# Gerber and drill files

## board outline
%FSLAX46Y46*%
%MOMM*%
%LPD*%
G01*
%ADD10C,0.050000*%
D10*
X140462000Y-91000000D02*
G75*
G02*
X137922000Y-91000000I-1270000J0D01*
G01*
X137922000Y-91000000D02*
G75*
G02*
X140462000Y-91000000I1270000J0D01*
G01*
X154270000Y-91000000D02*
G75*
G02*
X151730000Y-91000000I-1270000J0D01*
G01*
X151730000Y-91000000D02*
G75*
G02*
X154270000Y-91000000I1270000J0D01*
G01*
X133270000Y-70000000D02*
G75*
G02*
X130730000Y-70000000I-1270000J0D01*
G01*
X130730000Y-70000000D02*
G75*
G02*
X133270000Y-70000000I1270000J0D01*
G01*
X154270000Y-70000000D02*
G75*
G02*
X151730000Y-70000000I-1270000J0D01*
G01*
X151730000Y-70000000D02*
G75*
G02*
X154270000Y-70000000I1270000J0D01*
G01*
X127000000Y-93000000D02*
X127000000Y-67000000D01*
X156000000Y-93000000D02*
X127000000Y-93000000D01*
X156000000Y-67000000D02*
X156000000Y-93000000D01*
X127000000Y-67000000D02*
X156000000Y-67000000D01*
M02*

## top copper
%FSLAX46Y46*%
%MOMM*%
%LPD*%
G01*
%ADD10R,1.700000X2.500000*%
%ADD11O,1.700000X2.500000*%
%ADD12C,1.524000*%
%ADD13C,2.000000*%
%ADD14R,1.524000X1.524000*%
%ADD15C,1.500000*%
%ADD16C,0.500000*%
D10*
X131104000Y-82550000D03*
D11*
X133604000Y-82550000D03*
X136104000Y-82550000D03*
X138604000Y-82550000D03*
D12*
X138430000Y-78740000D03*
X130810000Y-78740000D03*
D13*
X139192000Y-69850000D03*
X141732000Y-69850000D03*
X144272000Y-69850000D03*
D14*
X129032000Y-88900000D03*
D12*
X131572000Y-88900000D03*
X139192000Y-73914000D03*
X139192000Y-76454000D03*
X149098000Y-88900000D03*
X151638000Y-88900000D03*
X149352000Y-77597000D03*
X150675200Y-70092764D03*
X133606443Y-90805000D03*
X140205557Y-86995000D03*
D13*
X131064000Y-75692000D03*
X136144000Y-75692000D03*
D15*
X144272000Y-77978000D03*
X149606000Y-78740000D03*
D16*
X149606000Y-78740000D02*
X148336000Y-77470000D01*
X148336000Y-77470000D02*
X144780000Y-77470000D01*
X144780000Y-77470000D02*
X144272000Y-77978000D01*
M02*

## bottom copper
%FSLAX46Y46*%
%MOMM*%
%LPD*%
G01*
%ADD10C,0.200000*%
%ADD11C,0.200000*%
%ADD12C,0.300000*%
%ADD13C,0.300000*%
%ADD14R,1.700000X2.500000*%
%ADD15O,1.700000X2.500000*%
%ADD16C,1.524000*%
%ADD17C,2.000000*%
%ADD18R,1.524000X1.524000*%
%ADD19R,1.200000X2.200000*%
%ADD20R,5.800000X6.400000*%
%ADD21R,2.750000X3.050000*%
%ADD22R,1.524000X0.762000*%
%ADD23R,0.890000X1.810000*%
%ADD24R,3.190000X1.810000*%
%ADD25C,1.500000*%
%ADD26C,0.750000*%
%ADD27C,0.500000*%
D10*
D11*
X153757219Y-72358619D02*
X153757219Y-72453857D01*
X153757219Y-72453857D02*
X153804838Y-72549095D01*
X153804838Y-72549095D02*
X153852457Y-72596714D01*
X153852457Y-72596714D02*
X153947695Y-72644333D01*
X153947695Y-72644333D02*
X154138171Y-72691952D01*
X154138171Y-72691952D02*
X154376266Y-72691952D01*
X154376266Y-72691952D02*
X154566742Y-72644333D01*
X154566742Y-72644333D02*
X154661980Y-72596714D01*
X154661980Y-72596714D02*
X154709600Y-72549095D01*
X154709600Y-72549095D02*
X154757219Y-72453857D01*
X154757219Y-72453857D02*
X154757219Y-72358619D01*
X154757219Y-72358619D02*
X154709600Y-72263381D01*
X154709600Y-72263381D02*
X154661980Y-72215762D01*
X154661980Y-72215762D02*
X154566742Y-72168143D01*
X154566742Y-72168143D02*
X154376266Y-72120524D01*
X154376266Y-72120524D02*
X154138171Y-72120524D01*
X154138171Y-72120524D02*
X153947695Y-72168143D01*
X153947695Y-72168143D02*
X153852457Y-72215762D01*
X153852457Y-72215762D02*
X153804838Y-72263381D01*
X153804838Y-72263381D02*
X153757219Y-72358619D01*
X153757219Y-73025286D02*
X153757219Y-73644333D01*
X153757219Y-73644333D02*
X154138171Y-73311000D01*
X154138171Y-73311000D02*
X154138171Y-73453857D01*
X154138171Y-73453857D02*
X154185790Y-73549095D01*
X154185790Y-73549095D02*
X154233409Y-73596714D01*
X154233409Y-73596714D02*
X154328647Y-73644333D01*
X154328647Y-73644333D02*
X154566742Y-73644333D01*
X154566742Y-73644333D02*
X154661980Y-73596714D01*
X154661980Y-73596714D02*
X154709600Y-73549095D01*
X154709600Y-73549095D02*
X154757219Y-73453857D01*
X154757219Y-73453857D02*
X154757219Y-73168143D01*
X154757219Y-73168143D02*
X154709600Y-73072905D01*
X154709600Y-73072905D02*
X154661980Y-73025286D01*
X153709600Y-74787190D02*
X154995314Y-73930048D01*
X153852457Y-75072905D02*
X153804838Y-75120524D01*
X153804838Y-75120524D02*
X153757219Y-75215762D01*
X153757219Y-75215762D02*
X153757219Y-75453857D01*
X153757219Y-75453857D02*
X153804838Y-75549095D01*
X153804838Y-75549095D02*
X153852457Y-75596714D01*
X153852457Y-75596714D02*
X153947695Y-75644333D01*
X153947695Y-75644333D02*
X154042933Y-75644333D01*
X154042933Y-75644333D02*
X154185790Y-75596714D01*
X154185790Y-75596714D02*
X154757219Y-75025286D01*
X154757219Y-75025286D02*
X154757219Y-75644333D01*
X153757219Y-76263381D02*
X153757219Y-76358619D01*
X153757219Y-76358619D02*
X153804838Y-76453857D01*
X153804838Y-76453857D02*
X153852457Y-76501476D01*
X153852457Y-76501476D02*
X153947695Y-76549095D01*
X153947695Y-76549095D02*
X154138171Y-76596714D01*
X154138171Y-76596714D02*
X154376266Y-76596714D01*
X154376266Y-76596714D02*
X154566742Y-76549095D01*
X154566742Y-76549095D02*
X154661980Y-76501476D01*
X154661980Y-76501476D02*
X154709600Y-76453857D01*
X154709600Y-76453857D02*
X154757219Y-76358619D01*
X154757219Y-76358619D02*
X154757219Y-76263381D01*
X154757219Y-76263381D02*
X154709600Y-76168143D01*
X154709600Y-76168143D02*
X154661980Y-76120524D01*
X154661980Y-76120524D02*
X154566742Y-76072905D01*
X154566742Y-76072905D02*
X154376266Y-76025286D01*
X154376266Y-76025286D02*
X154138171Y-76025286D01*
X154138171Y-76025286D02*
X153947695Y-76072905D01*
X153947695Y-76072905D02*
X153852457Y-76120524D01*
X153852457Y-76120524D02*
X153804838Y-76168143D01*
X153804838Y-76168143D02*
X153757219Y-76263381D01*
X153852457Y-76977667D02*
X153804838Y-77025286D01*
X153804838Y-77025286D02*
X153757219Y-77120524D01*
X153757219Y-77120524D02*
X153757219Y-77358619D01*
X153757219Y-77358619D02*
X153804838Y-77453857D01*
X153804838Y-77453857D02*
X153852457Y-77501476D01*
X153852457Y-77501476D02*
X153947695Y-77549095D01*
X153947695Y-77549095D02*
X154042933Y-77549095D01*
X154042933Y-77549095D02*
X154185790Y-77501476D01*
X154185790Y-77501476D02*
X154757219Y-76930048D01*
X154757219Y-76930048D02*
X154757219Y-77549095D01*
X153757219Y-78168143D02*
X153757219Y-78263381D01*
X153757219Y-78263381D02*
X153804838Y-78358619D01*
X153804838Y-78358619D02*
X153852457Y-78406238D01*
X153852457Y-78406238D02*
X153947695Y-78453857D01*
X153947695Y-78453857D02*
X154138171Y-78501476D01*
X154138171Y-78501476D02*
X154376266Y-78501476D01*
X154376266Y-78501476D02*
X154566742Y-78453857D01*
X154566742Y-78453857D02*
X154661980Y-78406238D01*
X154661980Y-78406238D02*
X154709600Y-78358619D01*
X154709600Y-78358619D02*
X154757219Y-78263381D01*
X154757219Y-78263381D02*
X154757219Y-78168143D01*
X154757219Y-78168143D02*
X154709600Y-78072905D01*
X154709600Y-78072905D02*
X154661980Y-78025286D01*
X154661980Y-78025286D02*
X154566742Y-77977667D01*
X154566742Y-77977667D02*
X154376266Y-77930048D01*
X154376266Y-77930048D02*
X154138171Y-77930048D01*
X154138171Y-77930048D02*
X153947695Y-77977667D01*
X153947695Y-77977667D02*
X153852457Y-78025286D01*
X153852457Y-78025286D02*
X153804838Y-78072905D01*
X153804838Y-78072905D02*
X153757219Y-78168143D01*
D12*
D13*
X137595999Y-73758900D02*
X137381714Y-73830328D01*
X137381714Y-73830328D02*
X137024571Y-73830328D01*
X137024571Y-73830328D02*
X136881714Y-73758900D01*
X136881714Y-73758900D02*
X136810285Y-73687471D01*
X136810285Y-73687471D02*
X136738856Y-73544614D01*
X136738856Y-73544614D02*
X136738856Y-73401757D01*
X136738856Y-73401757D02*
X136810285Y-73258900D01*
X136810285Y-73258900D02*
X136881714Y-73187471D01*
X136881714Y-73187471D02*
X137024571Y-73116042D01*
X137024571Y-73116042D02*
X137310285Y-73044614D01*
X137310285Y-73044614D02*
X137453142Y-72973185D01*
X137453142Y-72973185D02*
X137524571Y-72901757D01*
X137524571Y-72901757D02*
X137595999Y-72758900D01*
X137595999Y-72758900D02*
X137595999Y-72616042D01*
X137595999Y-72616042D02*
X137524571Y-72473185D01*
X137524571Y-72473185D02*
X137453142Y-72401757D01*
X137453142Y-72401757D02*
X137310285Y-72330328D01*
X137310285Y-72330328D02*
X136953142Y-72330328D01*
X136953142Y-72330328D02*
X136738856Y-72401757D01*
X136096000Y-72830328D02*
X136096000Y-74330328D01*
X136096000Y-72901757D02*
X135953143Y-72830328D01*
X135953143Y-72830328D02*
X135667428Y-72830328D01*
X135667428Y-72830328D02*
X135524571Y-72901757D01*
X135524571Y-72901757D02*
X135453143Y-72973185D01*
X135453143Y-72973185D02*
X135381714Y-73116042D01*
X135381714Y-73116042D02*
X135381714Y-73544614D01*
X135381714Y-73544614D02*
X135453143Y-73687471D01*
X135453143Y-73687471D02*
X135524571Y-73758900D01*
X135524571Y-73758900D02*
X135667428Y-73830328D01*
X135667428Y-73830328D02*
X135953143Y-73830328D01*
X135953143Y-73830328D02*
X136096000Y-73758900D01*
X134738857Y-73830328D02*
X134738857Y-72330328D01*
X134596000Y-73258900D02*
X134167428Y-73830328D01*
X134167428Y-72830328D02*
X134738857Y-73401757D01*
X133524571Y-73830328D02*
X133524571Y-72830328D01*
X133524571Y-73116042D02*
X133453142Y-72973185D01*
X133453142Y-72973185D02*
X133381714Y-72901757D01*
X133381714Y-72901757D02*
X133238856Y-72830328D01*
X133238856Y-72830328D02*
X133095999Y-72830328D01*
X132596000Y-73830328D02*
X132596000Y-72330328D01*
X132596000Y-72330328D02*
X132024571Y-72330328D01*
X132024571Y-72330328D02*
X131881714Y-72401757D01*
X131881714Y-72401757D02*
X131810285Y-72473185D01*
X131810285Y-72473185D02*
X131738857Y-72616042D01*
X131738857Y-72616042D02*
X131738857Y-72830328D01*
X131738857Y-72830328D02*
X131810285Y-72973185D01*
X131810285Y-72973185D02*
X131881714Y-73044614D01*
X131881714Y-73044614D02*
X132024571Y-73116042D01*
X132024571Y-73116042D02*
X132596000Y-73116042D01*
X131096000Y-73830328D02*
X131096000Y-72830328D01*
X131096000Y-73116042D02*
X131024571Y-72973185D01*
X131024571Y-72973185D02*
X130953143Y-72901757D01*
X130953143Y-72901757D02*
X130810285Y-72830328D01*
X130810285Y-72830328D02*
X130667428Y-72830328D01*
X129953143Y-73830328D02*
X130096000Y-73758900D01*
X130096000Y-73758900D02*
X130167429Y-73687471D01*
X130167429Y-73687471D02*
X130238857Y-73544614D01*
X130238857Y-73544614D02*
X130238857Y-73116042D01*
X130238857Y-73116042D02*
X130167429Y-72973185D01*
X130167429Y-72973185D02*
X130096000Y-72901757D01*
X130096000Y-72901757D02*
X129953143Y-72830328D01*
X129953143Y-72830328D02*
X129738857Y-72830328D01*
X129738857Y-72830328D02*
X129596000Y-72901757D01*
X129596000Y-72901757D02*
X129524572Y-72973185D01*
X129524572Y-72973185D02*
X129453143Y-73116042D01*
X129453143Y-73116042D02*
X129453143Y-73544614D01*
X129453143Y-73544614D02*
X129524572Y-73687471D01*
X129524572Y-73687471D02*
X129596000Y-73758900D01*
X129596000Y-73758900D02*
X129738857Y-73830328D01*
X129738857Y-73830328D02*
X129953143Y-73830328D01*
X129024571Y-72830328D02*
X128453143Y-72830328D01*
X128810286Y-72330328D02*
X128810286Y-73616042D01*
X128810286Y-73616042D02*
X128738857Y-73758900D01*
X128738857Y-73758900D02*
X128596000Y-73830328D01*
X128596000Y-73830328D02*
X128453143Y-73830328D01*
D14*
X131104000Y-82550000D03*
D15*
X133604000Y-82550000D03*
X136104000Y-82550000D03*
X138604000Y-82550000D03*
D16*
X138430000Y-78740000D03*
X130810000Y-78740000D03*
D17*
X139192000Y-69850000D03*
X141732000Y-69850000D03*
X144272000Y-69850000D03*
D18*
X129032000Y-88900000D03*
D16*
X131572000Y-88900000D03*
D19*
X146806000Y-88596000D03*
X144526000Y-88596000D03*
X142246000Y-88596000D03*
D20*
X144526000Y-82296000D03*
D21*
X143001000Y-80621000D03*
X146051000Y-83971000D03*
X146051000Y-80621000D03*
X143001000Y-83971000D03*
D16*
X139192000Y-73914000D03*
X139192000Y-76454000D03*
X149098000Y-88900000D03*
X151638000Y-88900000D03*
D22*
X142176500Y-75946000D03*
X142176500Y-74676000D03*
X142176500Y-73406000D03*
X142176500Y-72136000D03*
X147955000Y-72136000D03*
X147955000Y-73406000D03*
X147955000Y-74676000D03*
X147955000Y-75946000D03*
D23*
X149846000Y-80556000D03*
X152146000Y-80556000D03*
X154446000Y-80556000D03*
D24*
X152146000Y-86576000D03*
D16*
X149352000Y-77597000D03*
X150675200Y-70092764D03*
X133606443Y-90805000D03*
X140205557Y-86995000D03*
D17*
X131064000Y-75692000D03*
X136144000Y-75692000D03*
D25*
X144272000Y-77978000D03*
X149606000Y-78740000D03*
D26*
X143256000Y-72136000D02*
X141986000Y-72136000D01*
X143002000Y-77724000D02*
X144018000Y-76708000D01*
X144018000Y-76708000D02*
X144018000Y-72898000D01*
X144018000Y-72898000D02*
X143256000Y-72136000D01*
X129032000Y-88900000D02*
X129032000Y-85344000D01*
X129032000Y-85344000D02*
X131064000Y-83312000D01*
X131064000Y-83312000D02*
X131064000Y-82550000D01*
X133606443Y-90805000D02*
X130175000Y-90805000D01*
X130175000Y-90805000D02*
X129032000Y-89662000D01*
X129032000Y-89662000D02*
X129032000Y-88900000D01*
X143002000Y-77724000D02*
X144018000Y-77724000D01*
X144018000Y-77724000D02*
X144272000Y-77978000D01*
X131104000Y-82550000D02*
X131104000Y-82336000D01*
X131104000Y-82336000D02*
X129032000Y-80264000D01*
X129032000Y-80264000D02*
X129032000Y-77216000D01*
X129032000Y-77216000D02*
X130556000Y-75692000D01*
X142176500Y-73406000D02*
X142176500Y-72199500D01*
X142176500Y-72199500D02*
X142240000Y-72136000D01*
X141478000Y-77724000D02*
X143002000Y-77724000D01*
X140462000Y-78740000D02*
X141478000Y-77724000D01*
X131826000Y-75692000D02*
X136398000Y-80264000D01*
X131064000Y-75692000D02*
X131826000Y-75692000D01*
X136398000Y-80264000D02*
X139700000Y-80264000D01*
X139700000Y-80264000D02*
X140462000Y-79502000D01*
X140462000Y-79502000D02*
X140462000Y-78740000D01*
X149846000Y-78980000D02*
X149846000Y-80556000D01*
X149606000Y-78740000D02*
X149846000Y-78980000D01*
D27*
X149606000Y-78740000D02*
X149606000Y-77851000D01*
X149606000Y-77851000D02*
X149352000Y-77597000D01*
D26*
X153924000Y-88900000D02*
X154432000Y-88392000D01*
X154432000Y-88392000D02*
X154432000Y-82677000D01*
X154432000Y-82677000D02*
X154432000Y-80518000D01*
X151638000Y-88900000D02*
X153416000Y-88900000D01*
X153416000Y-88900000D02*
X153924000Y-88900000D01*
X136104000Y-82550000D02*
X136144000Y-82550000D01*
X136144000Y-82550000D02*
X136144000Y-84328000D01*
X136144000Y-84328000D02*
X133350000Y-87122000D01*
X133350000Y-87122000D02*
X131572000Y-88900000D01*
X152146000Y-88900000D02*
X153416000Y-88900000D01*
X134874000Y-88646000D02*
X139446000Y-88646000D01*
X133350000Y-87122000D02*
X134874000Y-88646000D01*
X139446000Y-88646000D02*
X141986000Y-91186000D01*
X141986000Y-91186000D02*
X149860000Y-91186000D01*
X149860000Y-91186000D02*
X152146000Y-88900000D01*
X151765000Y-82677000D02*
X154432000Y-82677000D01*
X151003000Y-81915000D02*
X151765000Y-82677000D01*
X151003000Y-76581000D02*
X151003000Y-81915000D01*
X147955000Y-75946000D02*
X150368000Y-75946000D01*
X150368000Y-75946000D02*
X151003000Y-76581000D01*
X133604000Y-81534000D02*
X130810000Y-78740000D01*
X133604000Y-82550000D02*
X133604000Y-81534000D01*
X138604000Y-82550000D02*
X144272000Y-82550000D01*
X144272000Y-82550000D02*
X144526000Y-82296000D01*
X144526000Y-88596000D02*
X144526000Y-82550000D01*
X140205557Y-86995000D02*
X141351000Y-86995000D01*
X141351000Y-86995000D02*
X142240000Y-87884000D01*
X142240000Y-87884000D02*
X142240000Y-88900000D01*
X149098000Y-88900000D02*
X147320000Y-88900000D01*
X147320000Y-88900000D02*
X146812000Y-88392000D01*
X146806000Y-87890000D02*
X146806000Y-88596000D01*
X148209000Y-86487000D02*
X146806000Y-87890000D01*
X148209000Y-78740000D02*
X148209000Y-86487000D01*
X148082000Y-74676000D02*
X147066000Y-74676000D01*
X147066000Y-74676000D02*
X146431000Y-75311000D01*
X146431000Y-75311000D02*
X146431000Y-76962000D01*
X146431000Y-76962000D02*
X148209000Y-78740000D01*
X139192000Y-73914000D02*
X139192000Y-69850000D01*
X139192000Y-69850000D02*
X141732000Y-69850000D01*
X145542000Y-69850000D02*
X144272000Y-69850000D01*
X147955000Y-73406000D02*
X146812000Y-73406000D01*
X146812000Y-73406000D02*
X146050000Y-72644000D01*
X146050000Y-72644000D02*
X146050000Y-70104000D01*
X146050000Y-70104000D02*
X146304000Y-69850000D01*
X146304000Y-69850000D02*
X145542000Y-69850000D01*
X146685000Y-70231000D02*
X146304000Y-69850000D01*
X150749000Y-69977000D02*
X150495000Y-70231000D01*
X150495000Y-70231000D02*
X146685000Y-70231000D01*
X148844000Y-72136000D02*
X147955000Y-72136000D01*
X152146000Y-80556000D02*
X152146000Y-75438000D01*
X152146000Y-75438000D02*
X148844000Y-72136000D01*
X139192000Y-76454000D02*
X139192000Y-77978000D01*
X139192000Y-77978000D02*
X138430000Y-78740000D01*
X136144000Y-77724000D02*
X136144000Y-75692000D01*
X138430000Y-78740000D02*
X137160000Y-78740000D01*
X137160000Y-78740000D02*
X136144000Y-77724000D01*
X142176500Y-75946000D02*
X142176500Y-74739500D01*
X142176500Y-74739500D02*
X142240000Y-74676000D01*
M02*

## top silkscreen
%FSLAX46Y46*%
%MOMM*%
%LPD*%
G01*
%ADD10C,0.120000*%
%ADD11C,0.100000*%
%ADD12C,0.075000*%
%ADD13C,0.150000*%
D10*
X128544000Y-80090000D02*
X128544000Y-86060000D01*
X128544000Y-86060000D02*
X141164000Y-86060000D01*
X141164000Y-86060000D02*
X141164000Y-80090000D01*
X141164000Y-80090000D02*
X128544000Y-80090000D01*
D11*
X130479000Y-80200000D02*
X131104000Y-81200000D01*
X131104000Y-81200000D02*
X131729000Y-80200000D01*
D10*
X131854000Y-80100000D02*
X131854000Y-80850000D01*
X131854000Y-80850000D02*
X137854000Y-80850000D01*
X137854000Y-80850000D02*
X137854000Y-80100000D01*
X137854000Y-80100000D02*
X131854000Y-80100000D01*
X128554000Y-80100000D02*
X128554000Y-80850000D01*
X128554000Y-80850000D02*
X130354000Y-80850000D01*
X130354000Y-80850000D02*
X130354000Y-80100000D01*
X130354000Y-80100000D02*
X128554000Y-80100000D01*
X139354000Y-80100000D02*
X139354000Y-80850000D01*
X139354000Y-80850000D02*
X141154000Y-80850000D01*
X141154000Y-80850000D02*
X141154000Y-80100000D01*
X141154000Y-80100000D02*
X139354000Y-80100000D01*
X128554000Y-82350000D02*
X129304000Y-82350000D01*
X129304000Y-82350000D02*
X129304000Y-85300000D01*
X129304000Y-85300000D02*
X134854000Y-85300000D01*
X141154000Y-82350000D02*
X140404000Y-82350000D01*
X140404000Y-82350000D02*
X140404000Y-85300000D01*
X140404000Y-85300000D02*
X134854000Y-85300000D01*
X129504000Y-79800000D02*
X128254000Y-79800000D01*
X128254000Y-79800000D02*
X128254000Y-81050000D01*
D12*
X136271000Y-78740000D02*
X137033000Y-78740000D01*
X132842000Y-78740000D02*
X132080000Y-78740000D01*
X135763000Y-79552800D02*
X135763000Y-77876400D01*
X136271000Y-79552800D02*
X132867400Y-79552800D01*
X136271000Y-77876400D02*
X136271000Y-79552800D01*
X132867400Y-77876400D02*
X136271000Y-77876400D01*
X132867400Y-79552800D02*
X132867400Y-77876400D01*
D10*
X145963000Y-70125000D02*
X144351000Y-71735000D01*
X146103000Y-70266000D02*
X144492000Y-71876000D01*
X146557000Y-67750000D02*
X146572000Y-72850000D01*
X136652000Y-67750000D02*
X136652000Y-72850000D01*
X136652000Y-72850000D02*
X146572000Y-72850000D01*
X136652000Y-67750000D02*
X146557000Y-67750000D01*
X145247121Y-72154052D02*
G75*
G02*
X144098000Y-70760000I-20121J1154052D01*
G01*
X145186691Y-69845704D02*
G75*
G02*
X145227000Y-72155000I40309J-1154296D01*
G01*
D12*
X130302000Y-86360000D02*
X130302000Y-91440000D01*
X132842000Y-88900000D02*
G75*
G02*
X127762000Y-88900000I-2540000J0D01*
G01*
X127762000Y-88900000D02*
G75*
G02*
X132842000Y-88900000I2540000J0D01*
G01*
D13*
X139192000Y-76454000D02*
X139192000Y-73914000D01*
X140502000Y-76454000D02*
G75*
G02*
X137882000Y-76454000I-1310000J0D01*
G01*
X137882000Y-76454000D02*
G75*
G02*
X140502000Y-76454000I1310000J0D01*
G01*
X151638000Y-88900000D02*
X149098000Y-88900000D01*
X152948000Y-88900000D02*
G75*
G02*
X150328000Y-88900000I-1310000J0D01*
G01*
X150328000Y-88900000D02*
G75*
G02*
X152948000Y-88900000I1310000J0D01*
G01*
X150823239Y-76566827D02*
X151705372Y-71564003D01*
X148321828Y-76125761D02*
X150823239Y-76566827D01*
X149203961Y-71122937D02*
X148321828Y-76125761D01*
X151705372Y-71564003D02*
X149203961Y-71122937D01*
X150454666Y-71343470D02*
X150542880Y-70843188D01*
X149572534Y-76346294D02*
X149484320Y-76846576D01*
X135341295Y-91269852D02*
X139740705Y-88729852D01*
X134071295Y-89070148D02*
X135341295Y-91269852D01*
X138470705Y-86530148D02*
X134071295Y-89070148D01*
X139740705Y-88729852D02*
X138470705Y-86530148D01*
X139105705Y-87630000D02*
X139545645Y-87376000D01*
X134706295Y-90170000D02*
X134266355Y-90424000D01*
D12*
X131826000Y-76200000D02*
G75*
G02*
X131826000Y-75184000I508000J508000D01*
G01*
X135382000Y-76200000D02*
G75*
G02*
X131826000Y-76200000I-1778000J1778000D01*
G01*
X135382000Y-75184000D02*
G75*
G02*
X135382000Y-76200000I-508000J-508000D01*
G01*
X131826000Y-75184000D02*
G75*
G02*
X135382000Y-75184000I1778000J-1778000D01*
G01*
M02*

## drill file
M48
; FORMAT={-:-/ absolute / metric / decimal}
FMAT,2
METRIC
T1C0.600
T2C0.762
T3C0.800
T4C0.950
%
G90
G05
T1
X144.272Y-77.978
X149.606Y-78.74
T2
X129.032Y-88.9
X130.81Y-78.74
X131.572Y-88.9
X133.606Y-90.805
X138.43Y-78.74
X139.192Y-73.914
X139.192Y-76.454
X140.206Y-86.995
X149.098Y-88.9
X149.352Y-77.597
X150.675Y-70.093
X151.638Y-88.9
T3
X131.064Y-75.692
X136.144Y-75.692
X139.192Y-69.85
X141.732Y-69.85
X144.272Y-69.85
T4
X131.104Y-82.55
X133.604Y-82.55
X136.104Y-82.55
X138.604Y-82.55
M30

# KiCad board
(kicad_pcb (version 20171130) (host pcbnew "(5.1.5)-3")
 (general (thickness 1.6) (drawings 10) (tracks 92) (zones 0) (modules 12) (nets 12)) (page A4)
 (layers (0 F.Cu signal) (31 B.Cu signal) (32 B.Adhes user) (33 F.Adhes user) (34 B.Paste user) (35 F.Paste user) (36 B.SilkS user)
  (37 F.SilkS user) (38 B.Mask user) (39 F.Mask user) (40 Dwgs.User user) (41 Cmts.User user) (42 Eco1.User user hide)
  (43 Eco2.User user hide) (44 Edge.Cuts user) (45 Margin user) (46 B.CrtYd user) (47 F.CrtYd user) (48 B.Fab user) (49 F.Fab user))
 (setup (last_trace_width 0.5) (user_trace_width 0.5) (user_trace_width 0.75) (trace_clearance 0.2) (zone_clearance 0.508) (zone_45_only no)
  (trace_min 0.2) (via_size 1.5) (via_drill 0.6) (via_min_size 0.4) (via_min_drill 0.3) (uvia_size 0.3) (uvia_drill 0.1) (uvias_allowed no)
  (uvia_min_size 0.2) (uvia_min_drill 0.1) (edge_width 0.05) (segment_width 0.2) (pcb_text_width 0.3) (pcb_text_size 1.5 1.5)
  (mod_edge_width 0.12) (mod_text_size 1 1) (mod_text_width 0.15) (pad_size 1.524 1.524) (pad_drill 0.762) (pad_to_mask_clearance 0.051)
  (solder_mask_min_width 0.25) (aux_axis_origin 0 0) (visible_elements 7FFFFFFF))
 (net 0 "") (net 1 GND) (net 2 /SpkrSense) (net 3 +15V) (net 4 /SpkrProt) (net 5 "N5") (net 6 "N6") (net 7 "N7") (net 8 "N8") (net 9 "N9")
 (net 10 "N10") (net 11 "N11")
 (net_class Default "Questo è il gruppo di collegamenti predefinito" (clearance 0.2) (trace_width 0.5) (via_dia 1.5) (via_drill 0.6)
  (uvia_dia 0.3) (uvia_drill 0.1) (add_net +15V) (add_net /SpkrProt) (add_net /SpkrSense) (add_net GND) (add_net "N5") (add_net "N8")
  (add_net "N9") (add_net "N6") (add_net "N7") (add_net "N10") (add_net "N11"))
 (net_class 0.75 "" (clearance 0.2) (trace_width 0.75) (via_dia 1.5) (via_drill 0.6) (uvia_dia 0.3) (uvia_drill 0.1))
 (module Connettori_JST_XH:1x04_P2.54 (layer F.Cu) (at 131.104 82.55)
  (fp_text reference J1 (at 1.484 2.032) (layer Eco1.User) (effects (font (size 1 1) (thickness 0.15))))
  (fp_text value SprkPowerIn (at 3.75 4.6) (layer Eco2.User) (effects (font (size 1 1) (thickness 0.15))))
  (fp_line (start -2.56 -2.46) (end -2.56 3.51) (layer F.SilkS) (width 0.12))
  (fp_line (start -2.56 3.51) (end 10.06 3.51) (layer F.SilkS) (width 0.12))
  (fp_line (start 10.06 3.51) (end 10.06 -2.46) (layer F.SilkS) (width 0.12))
  (fp_line (start 10.06 -2.46) (end -2.56 -2.46) (layer F.SilkS) (width 0.12))
  (fp_line (start -0.625 -2.35) (end 0 -1.35) (layer F.SilkS) (width 0.1))
  (fp_line (start 0 -1.35) (end 0.625 -2.35) (layer F.SilkS) (width 0.1))
  (fp_line (start 0.75 -2.45) (end 0.75 -1.7) (layer F.SilkS) (width 0.12))
  (fp_line (start 0.75 -1.7) (end 6.75 -1.7) (layer F.SilkS) (width 0.12))
  (fp_line (start 6.75 -1.7) (end 6.75 -2.45) (layer F.SilkS) (width 0.12))
  (fp_line (start 6.75 -2.45) (end 0.75 -2.45) (layer F.SilkS) (width 0.12))
  (fp_line (start -2.55 -2.45) (end -2.55 -1.7) (layer F.SilkS) (width 0.12))
  (fp_line (start -2.55 -1.7) (end -0.75 -1.7) (layer F.SilkS) (width 0.12))
  (fp_line (start -0.75 -1.7) (end -0.75 -2.45) (layer F.SilkS) (width 0.12))
  (fp_line (start -0.75 -2.45) (end -2.55 -2.45) (layer F.SilkS) (width 0.12))
  (fp_line (start 8.25 -2.45) (end 8.25 -1.7) (layer F.SilkS) (width 0.12))
  (fp_line (start 8.25 -1.7) (end 10.05 -1.7) (layer F.SilkS) (width 0.12))
  (fp_line (start 10.05 -1.7) (end 10.05 -2.45) (layer F.SilkS) (width 0.12))
  (fp_line (start 10.05 -2.45) (end 8.25 -2.45) (layer F.SilkS) (width 0.12))
  (fp_line (start -2.55 -0.2) (end -1.8 -0.2) (layer F.SilkS) (width 0.12))
  (fp_line (start -1.8 -0.2) (end -1.8 2.75) (layer F.SilkS) (width 0.12))
  (fp_line (start -1.8 2.75) (end 3.75 2.75) (layer F.SilkS) (width 0.12))
  (fp_line (start 10.05 -0.2) (end 9.3 -0.2) (layer F.SilkS) (width 0.12))
  (fp_line (start 9.3 -0.2) (end 9.3 2.75) (layer F.SilkS) (width 0.12))
  (fp_line (start 9.3 2.75) (end 3.75 2.75) (layer F.SilkS) (width 0.12))
  (fp_line (start -1.6 -2.75) (end -2.85 -2.75) (layer F.SilkS) (width 0.12))
  (fp_line (start -2.85 -2.75) (end -2.85 -1.5) (layer F.SilkS) (width 0.12))
  (pad 1 thru_hole rect (at 0 0) (size 1.7 2.5) (drill 0.95) (layers *.Cu *.Mask) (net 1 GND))
  (pad 2 thru_hole oval (at 2.5 0) (size 1.7 2.5) (drill 0.95) (layers *.Cu *.Mask) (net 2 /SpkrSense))
  (pad 3 thru_hole oval (at 5 0) (size 1.7 2.5) (drill 0.95) (layers *.Cu *.Mask) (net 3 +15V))
  (pad 4 thru_hole oval (at 7.5 0) (size 1.7 2.5) (drill 0.95) (layers *.Cu *.Mask) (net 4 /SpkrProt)))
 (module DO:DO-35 (layer F.Cu) (at 134.62 78.74 180)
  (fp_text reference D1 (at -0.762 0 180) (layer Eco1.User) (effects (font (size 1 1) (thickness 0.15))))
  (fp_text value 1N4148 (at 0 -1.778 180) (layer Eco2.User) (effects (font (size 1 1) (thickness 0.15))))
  (fp_line (start -1.651 0) (end -2.413 0) (layer F.SilkS) (width 0.075))
  (fp_line (start 1.778 0) (end 2.54 0) (layer F.SilkS) (width 0.075))
  (fp_line (start -1.143 -0.8128) (end -1.143 0.8636) (layer F.SilkS) (width 0.075))
  (fp_line (start -1.651 -0.8128) (end 1.7526 -0.8128) (layer F.SilkS) (width 0.075))
  (fp_line (start -1.651 0.8636) (end -1.651 -0.8128) (layer F.SilkS) (width 0.075))
  (fp_line (start 1.7526 0.8636) (end -1.651 0.8636) (layer F.SilkS) (width 0.075))
  (fp_line (start 1.7526 -0.8128) (end 1.7526 0.8636) (layer F.SilkS) (width 0.075))
  (pad 1 thru_hole circle (at -3.81 0 180) (size 1.524 1.524) (drill 0.762) (layers *.Cu *.Mask) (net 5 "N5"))
  (pad 2 thru_hole circle (at 3.81 0 180) (size 1.524 1.524) (drill 0.762) (layers *.Cu *.Mask) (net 2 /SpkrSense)))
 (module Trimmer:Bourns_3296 (layer F.Cu) (at 144.272 69.85)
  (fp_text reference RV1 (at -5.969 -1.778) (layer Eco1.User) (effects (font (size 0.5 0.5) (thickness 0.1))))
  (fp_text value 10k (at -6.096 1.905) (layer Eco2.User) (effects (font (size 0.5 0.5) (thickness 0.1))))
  (fp_line (start 1.691 0.275) (end 0.079 1.885) (layer F.SilkS) (width 0.12))
  (fp_line (start 1.831 0.416) (end 0.22 2.026) (layer F.SilkS) (width 0.12))
  (fp_line (start 2.285 -2.1) (end 2.3 3) (layer F.SilkS) (width 0.12))
  (fp_line (start -7.62 -2.1) (end -7.62 3) (layer F.SilkS) (width 0.12))
  (fp_line (start -7.62 3) (end 2.3 3) (layer F.SilkS) (width 0.12))
  (fp_line (start -7.62 -2.1) (end 2.285 -2.1) (layer F.SilkS) (width 0.12))
  (fp_arc (start 0.955 1.15) (end -0.174 0.91) (angle -103) (layer F.SilkS) (width 0.12))
  (fp_arc (start 0.955 1.15) (end 0.955 2.305) (angle -182) (layer F.SilkS) (width 0.12))
  (pad 3 thru_hole circle (at -5.08 0) (size 2 2) (drill 0.8) (layers *.Cu *.Mask) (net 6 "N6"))
  (pad 2 thru_hole circle (at -2.54 0) (size 2 2) (drill 0.8) (layers *.Cu *.Mask) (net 6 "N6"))
  (pad 1 thru_hole circle (at 0 0) (size 2 2) (drill 0.8) (layers *.Cu *.Mask) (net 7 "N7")))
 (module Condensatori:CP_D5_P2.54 (layer F.Cu) (at 130.302 88.9)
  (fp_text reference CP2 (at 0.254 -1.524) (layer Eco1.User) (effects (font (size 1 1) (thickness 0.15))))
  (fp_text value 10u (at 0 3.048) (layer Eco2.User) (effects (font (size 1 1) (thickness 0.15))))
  (fp_line (start 0 -2.54) (end 0 2.54) (layer F.SilkS) (width 0.075))
  (fp_circle (center 0 0) (end 2.54 0) (layer F.SilkS) (width 0.075))
  (pad 1 thru_hole rect (at -1.27 0) (size 1.524 1.524) (drill 0.762) (layers *.Cu *.Mask) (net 1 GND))
  (pad 2 thru_hole circle (at 1.27 0) (size 1.524 1.524) (drill 0.762) (layers *.Cu *.Mask) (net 3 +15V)))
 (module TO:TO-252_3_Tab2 (layer B.Cu) (at 144.526 84.396 90)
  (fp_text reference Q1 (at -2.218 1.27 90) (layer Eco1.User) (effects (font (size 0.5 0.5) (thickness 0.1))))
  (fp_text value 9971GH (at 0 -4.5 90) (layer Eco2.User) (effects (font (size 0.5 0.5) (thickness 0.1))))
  (pad 1 smd rect (at -4.2 2.28 90) (size 2.2 1.2) (layers B.Cu B.Paste B.Mask) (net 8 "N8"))
  (pad 2 smd rect (at -4.2 0 90) (size 2.2 1.2) (layers B.Cu B.Paste B.Mask) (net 4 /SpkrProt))
  (pad 3 smd rect (at -4.2 -2.28 90) (size 2.2 1.2) (layers B.Cu B.Paste B.Mask) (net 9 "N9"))
  (pad 2 smd rect (at 2.1 0 90) (size 6.4 5.8) (layers B.Cu B.Mask) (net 4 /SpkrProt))
  (pad 2 smd rect (at 3.775 -1.525 90) (size 3.05 2.75) (layers B.Cu B.Paste) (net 4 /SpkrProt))
  (pad 2 smd rect (at 0.425 1.525 90) (size 3.05 2.75) (layers B.Cu B.Paste) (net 4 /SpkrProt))
  (pad 2 smd rect (at 3.775 1.525 90) (size 3.05 2.75) (layers B.Cu B.Paste) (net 4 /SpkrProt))
  (pad 2 smd rect (at 0.425 -1.525 90) (size 3.05 2.75) (layers B.Cu B.Paste) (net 4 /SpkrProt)))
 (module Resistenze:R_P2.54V (layer F.Cu) (at 139.192 76.454 90)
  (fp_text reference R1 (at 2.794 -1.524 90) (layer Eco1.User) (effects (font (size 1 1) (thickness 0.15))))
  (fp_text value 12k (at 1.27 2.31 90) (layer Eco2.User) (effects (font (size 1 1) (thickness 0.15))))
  (fp_line (start 0 0) (end 2.54 0) (layer F.SilkS) (width 0.15))
  (fp_circle (center 0 0) (end 1.31 0) (layer F.SilkS) (width 0.15))
  (pad 2 thru_hole circle (at 2.54 0 90) (size 1.524 1.524) (drill 0.762) (layers *.Cu *.Mask) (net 6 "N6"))
  (pad 1 thru_hole circle (at 0 0 90) (size 1.524 1.524) (drill 0.762) (layers *.Cu *.Mask) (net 5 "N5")))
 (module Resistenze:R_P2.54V (layer F.Cu) (at 151.638 88.9 180)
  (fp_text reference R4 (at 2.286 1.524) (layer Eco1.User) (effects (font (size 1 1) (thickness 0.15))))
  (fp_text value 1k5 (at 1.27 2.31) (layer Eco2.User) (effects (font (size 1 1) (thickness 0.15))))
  (fp_line (start 0 0) (end 2.54 0) (layer F.SilkS) (width 0.15))
  (fp_circle (center 0 0) (end 1.31 0) (layer F.SilkS) (width 0.15))
  (pad 2 thru_hole circle (at 2.54 0 180) (size 1.524 1.524) (drill 0.762) (layers *.Cu *.Mask) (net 8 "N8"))
  (pad 1 thru_hole circle (at 0 0 180) (size 1.524 1.524) (drill 0.762) (layers *.Cu *.Mask) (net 3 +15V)))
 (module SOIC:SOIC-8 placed (layer B.Cu) (at 145.034 72.136 90)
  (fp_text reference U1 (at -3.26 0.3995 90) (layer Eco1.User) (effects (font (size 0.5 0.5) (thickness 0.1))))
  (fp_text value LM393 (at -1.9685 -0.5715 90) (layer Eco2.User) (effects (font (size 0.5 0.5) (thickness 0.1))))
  (pad 1 smd rect (at -3.81 -2.8575 90) (size 0.762 1.524) (layers B.Cu B.Paste B.Mask) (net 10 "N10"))
  (pad 2 smd rect (at -2.54 -2.8575 90) (size 0.762 1.524) (layers B.Cu B.Paste B.Mask) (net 10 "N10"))
  (pad 3 smd rect (at -1.27 -2.8575 90) (size 0.762 1.524) (layers B.Cu B.Paste B.Mask) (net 1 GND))
  (pad 4 smd rect (at 0 -2.8575 90) (size 0.762 1.524) (layers B.Cu B.Paste B.Mask) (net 1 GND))
  (pad 5 smd rect (at 0 2.921 90) (size 0.762 1.524) (layers B.Cu B.Paste B.Mask) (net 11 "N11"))
  (pad 6 smd rect (at -1.27 2.921 90) (size 0.762 1.524) (layers B.Cu B.Paste B.Mask) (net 7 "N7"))
  (pad 7 smd rect (at -2.54 2.921 90) (size 0.762 1.524) (layers B.Cu B.Paste B.Mask) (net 8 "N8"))
  (pad 8 smd rect (at -3.81 2.921 90) (size 0.762 1.524) (layers B.Cu B.Paste B.Mask) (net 3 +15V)))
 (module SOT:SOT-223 (layer B.Cu) (at 152.146 83.566 270)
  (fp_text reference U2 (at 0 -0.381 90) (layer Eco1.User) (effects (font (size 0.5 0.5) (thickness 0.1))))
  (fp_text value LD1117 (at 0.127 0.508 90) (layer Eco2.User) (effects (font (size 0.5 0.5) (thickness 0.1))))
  (pad 1 smd rect (at -3.01 2.3 270) (size 1.81 0.89) (layers B.Cu B.Paste B.Mask) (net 1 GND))
  (pad 2 smd rect (at -3.01 0 270) (size 1.81 0.89) (layers B.Cu B.Paste B.Mask) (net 11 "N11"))
  (pad 3 smd rect (at -3.01 -2.3 270) (size 1.81 0.89) (layers B.Cu B.Paste B.Mask) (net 3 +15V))
  (pad 4 smd rect (at 3.01 0 270) (size 1.81 3.19) (layers B.Cu B.Paste B.Mask)))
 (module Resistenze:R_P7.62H (layer F.Cu) (at 150.0136 73.844882 260)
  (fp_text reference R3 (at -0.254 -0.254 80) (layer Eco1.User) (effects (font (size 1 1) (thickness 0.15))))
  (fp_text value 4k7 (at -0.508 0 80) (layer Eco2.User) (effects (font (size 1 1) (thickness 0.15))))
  (fp_line (start 2.54 -1.27) (end -2.54 -1.27) (layer F.SilkS) (width 0.15))
  (fp_line (start 2.54 1.27) (end 2.54 -1.27) (layer F.SilkS) (width 0.15))
  (fp_line (start -2.54 1.27) (end 2.54 1.27) (layer F.SilkS) (width 0.15))
  (fp_line (start -2.54 -1.27) (end -2.54 1.27) (layer F.SilkS) (width 0.15))
  (fp_line (start -2.54 0) (end -3.048 0) (layer F.SilkS) (width 0.15))
  (fp_line (start 2.54 0) (end 3.048 0) (layer F.SilkS) (width 0.15))
  (pad 2 thru_hole circle (at 3.81 0 260) (size 1.524 1.524) (drill 0.762) (layers *.Cu *.Mask) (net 1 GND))
  (pad 1 thru_hole circle (at -3.81 0 260) (size 1.524 1.524) (drill 0.762) (layers *.Cu *.Mask) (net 7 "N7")))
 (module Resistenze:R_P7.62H (layer F.Cu) (at 136.906 88.9 210)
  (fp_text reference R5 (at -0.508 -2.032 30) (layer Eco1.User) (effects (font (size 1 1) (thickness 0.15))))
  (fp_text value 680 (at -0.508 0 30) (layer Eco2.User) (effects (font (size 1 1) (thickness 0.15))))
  (fp_line (start 2.54 -1.27) (end -2.54 -1.27) (layer F.SilkS) (width 0.15))
  (fp_line (start 2.54 1.27) (end 2.54 -1.27) (layer F.SilkS) (width 0.15))
  (fp_line (start -2.54 1.27) (end 2.54 1.27) (layer F.SilkS) (width 0.15))
  (fp_line (start -2.54 -1.27) (end -2.54 1.27) (layer F.SilkS) (width 0.15))
  (fp_line (start -2.54 0) (end -3.048 0) (layer F.SilkS) (width 0.15))
  (fp_line (start 2.54 0) (end 3.048 0) (layer F.SilkS) (width 0.15))
  (pad 2 thru_hole circle (at 3.81 0 210) (size 1.524 1.524) (drill 0.762) (layers *.Cu *.Mask) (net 1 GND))
  (pad 1 thru_hole circle (at -3.81 0 210) (size 1.524 1.524) (drill 0.762) (layers *.Cu *.Mask) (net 9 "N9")))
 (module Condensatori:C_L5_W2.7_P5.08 (layer F.Cu) (at 131.064 75.692)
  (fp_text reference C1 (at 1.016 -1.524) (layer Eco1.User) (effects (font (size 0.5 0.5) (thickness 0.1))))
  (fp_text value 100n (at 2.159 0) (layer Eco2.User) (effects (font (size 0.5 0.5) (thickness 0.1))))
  (fp_arc (start 1.27 0) (end 0.762 0.508) (angle 90) (layer F.SilkS) (width 0.075))
  (fp_arc (start 2.54 -1.27) (end 4.318 0.508) (angle 90) (layer F.SilkS) (width 0.075))
  (fp_arc (start 3.81 0) (end 4.318 -0.508) (angle 90) (layer F.SilkS) (width 0.075))
  (fp_arc (start 2.54 1.27) (end 0.762 -0.508) (angle 90) (layer F.SilkS) (width 0.075))
  (pad 1 thru_hole circle (at 0 0) (size 2 2) (drill 0.8) (layers *.Cu *.Mask) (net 1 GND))
  (pad 2 thru_hole circle (at 5.08 0) (size 2 2) (drill 0.8) (layers *.Cu *.Mask) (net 5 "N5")))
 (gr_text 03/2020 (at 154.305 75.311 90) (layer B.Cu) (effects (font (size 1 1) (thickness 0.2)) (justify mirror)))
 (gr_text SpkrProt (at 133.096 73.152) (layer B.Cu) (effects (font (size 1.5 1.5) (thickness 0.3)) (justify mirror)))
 (gr_circle (center 139.192 91) (end 140.462 91) (layer Edge.Cuts) (width 0.05))
 (gr_circle (center 153 91) (end 154.27 91) (layer Edge.Cuts) (width 0.05))
 (gr_circle (center 132 70) (end 133.27 70) (layer Edge.Cuts) (width 0.05))
 (gr_circle (center 153 70) (end 154.27 70) (layer Edge.Cuts) (width 0.05))
 (gr_line (start 127 93) (end 127 67) (layer Edge.Cuts) (width 0.05))
 (gr_line (start 156 93) (end 127 93) (layer Edge.Cuts) (width 0.05))
 (gr_line (start 156 67) (end 156 93) (layer Edge.Cuts) (width 0.05))
 (gr_line (start 127 67) (end 156 67) (layer Edge.Cuts) (width 0.05))
 (segment (start 143.256 72.136) (end 141.986 72.136) (width 0.75) (layer B.Cu) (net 1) (status 20))
 (segment (start 143.002 77.724) (end 144.018 76.708) (width 0.75) (layer B.Cu) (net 1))
 (segment (start 144.018 76.708) (end 144.018 72.898) (width 0.75) (layer B.Cu) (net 1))
 (segment (start 144.018 72.898) (end 143.256 72.136) (width 0.75) (layer B.Cu) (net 1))
 (segment (start 129.032 88.9) (end 129.032 85.344) (width 0.75) (layer B.Cu) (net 1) (status 10))
 (segment (start 129.032 85.344) (end 131.064 83.312) (width 0.75) (layer B.Cu) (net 1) (status 20))
 (segment (start 131.064 83.312) (end 131.064 82.55) (width 0.75) (layer B.Cu) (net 1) (status 30))
 (segment (start 133.606443 90.805) (end 130.175 90.805) (width 0.75) (layer B.Cu) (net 1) (status 10))
 (segment (start 130.175 90.805) (end 129.032 89.662) (width 0.75) (layer B.Cu) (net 1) (status 20))
 (segment (start 129.032 89.662) (end 129.032 88.9) (width 0.75) (layer B.Cu) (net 1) (status 30))
 (via (at 144.272 77.978) (size 1.5) (drill 0.6) (layers F.Cu B.Cu) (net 1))
 (segment (start 143.002 77.724) (end 144.018 77.724) (width 0.75) (layer B.Cu) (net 1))
 (segment (start 144.018 77.724) (end 144.272 77.978) (width 0.75) (layer B.Cu) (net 1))
 (segment (start 131.104 82.55) (end 131.104 82.336) (width 0.75) (layer B.Cu) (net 1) (status 30))
 (segment (start 131.104 82.336) (end 129.032 80.264) (width 0.75) (layer B.Cu) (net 1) (status 10))
 (segment (start 129.032 80.264) (end 129.032 77.216) (width 0.75) (layer B.Cu) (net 1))
 (segment (start 129.032 77.216) (end 130.556 75.692) (width 0.75) (layer B.Cu) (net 1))
 (segment (start 142.1765 73.406) (end 142.1765 72.1995) (width 0.75) (layer B.Cu) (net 1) (status 30))
 (segment (start 142.1765 72.1995) (end 142.24 72.136) (width 0.75) (layer B.Cu) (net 1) (status 30))
 (segment (start 141.478 77.724) (end 143.002 77.724) (width 0.75) (layer B.Cu) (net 1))
 (segment (start 140.462 78.74) (end 141.478 77.724) (width 0.75) (layer B.Cu) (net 1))
 (segment (start 131.826 75.692) (end 136.398 80.264) (width 0.75) (layer B.Cu) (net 1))
 (segment (start 131.064 75.692) (end 131.826 75.692) (width 0.75) (layer B.Cu) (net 1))
 (segment (start 136.398 80.264) (end 139.7 80.264) (width 0.75) (layer B.Cu) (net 1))
 (segment (start 139.7 80.264) (end 140.462 79.502) (width 0.75) (layer B.Cu) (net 1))
 (segment (start 140.462 79.502) (end 140.462 78.74) (width 0.75) (layer B.Cu) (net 1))
 (segment (start 149.846 78.98) (end 149.846 80.556) (width 0.75) (layer B.Cu) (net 1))
 (segment (start 149.606 78.74) (end 148.336 77.47) (width 0.5) (layer F.Cu) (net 1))
 (via (at 149.606 78.74) (size 1.5) (drill 0.6) (layers F.Cu B.Cu) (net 1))
 (segment (start 148.336 77.47) (end 144.78 77.47) (width 0.5) (layer F.Cu) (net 1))
 (segment (start 144.78 77.47) (end 144.272 77.978) (width 0.5) (layer F.Cu) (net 1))
 (segment (start 149.606 78.74) (end 149.846 78.98) (width 0.75) (layer B.Cu) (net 1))
 (segment (start 149.606 78.74) (end 149.606 77.851) (width 0.5) (layer B.Cu) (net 1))
 (segment (start 149.606 77.851) (end 149.352 77.597) (width 0.5) (layer B.Cu) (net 1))
 (segment (start 153.924 88.9) (end 154.432 88.392) (width 0.75) (layer B.Cu) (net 3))
 (segment (start 154.432 88.392) (end 154.432 82.677) (width 0.75) (layer B.Cu) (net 3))
 (segment (start 154.432 82.677) (end 154.432 80.518) (width 0.75) (layer B.Cu) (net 3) (status 20))
 (segment (start 151.638 88.9) (end 153.416 88.9) (width 0.75) (layer B.Cu) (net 3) (status 10))
 (segment (start 153.416 88.9) (end 153.924 88.9) (width 0.75) (layer B.Cu) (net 3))
 (segment (start 136.104 82.55) (end 136.144 82.55) (width 0.75) (layer B.Cu) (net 3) (status 30))
 (segment (start 136.144 82.55) (end 136.144 84.328) (width 0.75) (layer B.Cu) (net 3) (status 10))
 (segment (start 136.144 84.328) (end 133.35 87.122) (width 0.75) (layer B.Cu) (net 3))
 (segment (start 133.35 87.122) (end 131.572 88.9) (width 0.75) (layer B.Cu) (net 3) (status 20))
 (segment (start 152.146 88.9) (end 153.416 88.9) (width 0.75) (layer B.Cu) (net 3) (status 10))
 (segment (start 134.874 88.646) (end 139.446 88.646) (width 0.75) (layer B.Cu) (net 3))
 (segment (start 133.35 87.122) (end 134.874 88.646) (width 0.75) (layer B.Cu) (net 3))
 (segment (start 139.446 88.646) (end 141.986 91.186) (width 0.75) (layer B.Cu) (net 3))
 (segment (start 141.986 91.186) (end 149.86 91.186) (width 0.75) (layer B.Cu) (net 3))
 (segment (start 149.86 91.186) (end 152.146 88.9) (width 0.75) (layer B.Cu) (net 3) (status 20))
 (segment (start 151.765 82.677) (end 154.432 82.677) (width 0.75) (layer B.Cu) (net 3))
 (segment (start 151.003 81.915) (end 151.765 82.677) (width 0.75) (layer B.Cu) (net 3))
 (segment (start 151.003 76.581) (end 151.003 81.915) (width 0.75) (layer B.Cu) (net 3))
 (segment (start 147.955 75.946) (end 150.368 75.946) (width 0.75) (layer B.Cu) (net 3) (status 10))
 (segment (start 150.368 75.946) (end 151.003 76.581) (width 0.75) (layer B.Cu) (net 3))
 (segment (start 133.604 81.534) (end 130.81 78.74) (width 0.75) (layer B.Cu) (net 2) (status 30))
 (segment (start 133.604 82.55) (end 133.604 81.534) (width 0.75) (layer B.Cu) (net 2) (status 30))
 (segment (start 138.604 82.55) (end 144.272 82.55) (width 0.75) (layer B.Cu) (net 4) (status 30))
 (segment (start 144.272 82.55) (end 144.526 82.296) (width 0.75) (layer B.Cu) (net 4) (status 30))
 (segment (start 144.526 88.596) (end 144.526 82.55) (width 0.75) (layer B.Cu) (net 4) (status 30))
 (segment (start 140.205557 86.995) (end 141.351 86.995) (width 0.75) (layer B.Cu) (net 9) (status 10))
 (segment (start 141.351 86.995) (end 142.24 87.884) (width 0.75) (layer B.Cu) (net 9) (status 20))
 (segment (start 142.24 87.884) (end 142.24 88.9) (width 0.75) (layer B.Cu) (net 9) (status 30))
 (segment (start 149.098 88.9) (end 147.32 88.9) (width 0.75) (layer B.Cu) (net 8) (status 30))
 (segment (start 147.32 88.9) (end 146.812 88.392) (width 0.75) (layer B.Cu) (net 8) (status 30))
 (segment (start 146.806 87.89) (end 146.806 88.596) (width 0.75) (layer B.Cu) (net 8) (status 30))
 (segment (start 148.209 86.487) (end 146.806 87.89) (width 0.75) (layer B.Cu) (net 8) (status 20))
 (segment (start 148.209 78.74) (end 148.209 86.487) (width 0.75) (layer B.Cu) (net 8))
 (segment (start 148.082 74.676) (end 147.066 74.676) (width 0.75) (layer B.Cu) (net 8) (status 10))
 (segment (start 147.066 74.676) (end 146.431 75.311) (width 0.75) (layer B.Cu) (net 8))
 (segment (start 146.431 75.311) (end 146.431 76.962) (width 0.75) (layer B.Cu) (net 8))
 (segment (start 146.431 76.962) (end 148.209 78.74) (width 0.75) (layer B.Cu) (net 8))
 (segment (start 139.192 73.914) (end 139.192 69.85) (width 0.75) (layer B.Cu) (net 6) (status 30))
 (segment (start 139.192 69.85) (end 141.732 69.85) (width 0.75) (layer B.Cu) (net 6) (status 30))
 (segment (start 145.542 69.85) (end 144.272 69.85) (width 0.75) (layer B.Cu) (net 7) (status 20))
 (segment (start 147.955 73.406) (end 146.812 73.406) (width 0.75) (layer B.Cu) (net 7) (status 10))
 (segment (start 146.812 73.406) (end 146.05 72.644) (width 0.75) (layer B.Cu) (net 7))
 (segment (start 146.05 72.644) (end 146.05 70.104) (width 0.75) (layer B.Cu) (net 7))
 (segment (start 146.05 70.104) (end 146.304 69.85) (width 0.75) (layer B.Cu) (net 7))
 (segment (start 146.304 69.85) (end 145.542 69.85) (width 0.75) (layer B.Cu) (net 7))
 (segment (start 146.685 70.231) (end 146.304 69.85) (width 0.75) (layer B.Cu) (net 7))
 (segment (start 150.749 69.977) (end 150.495 70.231) (width 0.75) (layer B.Cu) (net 7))
 (segment (start 150.495 70.231) (end 146.685 70.231) (width 0.75) (layer B.Cu) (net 7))
 (segment (start 148.844 72.136) (end 147.955 72.136) (width 0.75) (layer B.Cu) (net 11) (status 20))
 (segment (start 152.146 80.556) (end 152.146 75.438) (width 0.75) (layer B.Cu) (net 11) (status 10))
 (segment (start 152.146 75.438) (end 148.844 72.136) (width 0.75) (layer B.Cu) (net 11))
 (segment (start 139.192 76.454) (end 139.192 77.978) (width 0.75) (layer B.Cu) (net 5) (status 10))
 (segment (start 139.192 77.978) (end 138.43 78.74) (width 0.75) (layer B.Cu) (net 5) (status 20))
 (segment (start 136.144 77.724) (end 136.144 75.692) (width 0.75) (layer B.Cu) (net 5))
 (segment (start 138.43 78.74) (end 137.16 78.74) (width 0.75) (layer B.Cu) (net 5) (status 10))
 (segment (start 137.16 78.74) (end 136.144 77.724) (width 0.75) (layer B.Cu) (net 5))
 (segment (start 142.1765 75.946) (end 142.1765 74.7395) (width 0.75) (layer B.Cu) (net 10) (status 30))
 (segment (start 142.1765 74.7395) (end 142.24 74.676) (width 0.75) (layer B.Cu) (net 10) (status 30)))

